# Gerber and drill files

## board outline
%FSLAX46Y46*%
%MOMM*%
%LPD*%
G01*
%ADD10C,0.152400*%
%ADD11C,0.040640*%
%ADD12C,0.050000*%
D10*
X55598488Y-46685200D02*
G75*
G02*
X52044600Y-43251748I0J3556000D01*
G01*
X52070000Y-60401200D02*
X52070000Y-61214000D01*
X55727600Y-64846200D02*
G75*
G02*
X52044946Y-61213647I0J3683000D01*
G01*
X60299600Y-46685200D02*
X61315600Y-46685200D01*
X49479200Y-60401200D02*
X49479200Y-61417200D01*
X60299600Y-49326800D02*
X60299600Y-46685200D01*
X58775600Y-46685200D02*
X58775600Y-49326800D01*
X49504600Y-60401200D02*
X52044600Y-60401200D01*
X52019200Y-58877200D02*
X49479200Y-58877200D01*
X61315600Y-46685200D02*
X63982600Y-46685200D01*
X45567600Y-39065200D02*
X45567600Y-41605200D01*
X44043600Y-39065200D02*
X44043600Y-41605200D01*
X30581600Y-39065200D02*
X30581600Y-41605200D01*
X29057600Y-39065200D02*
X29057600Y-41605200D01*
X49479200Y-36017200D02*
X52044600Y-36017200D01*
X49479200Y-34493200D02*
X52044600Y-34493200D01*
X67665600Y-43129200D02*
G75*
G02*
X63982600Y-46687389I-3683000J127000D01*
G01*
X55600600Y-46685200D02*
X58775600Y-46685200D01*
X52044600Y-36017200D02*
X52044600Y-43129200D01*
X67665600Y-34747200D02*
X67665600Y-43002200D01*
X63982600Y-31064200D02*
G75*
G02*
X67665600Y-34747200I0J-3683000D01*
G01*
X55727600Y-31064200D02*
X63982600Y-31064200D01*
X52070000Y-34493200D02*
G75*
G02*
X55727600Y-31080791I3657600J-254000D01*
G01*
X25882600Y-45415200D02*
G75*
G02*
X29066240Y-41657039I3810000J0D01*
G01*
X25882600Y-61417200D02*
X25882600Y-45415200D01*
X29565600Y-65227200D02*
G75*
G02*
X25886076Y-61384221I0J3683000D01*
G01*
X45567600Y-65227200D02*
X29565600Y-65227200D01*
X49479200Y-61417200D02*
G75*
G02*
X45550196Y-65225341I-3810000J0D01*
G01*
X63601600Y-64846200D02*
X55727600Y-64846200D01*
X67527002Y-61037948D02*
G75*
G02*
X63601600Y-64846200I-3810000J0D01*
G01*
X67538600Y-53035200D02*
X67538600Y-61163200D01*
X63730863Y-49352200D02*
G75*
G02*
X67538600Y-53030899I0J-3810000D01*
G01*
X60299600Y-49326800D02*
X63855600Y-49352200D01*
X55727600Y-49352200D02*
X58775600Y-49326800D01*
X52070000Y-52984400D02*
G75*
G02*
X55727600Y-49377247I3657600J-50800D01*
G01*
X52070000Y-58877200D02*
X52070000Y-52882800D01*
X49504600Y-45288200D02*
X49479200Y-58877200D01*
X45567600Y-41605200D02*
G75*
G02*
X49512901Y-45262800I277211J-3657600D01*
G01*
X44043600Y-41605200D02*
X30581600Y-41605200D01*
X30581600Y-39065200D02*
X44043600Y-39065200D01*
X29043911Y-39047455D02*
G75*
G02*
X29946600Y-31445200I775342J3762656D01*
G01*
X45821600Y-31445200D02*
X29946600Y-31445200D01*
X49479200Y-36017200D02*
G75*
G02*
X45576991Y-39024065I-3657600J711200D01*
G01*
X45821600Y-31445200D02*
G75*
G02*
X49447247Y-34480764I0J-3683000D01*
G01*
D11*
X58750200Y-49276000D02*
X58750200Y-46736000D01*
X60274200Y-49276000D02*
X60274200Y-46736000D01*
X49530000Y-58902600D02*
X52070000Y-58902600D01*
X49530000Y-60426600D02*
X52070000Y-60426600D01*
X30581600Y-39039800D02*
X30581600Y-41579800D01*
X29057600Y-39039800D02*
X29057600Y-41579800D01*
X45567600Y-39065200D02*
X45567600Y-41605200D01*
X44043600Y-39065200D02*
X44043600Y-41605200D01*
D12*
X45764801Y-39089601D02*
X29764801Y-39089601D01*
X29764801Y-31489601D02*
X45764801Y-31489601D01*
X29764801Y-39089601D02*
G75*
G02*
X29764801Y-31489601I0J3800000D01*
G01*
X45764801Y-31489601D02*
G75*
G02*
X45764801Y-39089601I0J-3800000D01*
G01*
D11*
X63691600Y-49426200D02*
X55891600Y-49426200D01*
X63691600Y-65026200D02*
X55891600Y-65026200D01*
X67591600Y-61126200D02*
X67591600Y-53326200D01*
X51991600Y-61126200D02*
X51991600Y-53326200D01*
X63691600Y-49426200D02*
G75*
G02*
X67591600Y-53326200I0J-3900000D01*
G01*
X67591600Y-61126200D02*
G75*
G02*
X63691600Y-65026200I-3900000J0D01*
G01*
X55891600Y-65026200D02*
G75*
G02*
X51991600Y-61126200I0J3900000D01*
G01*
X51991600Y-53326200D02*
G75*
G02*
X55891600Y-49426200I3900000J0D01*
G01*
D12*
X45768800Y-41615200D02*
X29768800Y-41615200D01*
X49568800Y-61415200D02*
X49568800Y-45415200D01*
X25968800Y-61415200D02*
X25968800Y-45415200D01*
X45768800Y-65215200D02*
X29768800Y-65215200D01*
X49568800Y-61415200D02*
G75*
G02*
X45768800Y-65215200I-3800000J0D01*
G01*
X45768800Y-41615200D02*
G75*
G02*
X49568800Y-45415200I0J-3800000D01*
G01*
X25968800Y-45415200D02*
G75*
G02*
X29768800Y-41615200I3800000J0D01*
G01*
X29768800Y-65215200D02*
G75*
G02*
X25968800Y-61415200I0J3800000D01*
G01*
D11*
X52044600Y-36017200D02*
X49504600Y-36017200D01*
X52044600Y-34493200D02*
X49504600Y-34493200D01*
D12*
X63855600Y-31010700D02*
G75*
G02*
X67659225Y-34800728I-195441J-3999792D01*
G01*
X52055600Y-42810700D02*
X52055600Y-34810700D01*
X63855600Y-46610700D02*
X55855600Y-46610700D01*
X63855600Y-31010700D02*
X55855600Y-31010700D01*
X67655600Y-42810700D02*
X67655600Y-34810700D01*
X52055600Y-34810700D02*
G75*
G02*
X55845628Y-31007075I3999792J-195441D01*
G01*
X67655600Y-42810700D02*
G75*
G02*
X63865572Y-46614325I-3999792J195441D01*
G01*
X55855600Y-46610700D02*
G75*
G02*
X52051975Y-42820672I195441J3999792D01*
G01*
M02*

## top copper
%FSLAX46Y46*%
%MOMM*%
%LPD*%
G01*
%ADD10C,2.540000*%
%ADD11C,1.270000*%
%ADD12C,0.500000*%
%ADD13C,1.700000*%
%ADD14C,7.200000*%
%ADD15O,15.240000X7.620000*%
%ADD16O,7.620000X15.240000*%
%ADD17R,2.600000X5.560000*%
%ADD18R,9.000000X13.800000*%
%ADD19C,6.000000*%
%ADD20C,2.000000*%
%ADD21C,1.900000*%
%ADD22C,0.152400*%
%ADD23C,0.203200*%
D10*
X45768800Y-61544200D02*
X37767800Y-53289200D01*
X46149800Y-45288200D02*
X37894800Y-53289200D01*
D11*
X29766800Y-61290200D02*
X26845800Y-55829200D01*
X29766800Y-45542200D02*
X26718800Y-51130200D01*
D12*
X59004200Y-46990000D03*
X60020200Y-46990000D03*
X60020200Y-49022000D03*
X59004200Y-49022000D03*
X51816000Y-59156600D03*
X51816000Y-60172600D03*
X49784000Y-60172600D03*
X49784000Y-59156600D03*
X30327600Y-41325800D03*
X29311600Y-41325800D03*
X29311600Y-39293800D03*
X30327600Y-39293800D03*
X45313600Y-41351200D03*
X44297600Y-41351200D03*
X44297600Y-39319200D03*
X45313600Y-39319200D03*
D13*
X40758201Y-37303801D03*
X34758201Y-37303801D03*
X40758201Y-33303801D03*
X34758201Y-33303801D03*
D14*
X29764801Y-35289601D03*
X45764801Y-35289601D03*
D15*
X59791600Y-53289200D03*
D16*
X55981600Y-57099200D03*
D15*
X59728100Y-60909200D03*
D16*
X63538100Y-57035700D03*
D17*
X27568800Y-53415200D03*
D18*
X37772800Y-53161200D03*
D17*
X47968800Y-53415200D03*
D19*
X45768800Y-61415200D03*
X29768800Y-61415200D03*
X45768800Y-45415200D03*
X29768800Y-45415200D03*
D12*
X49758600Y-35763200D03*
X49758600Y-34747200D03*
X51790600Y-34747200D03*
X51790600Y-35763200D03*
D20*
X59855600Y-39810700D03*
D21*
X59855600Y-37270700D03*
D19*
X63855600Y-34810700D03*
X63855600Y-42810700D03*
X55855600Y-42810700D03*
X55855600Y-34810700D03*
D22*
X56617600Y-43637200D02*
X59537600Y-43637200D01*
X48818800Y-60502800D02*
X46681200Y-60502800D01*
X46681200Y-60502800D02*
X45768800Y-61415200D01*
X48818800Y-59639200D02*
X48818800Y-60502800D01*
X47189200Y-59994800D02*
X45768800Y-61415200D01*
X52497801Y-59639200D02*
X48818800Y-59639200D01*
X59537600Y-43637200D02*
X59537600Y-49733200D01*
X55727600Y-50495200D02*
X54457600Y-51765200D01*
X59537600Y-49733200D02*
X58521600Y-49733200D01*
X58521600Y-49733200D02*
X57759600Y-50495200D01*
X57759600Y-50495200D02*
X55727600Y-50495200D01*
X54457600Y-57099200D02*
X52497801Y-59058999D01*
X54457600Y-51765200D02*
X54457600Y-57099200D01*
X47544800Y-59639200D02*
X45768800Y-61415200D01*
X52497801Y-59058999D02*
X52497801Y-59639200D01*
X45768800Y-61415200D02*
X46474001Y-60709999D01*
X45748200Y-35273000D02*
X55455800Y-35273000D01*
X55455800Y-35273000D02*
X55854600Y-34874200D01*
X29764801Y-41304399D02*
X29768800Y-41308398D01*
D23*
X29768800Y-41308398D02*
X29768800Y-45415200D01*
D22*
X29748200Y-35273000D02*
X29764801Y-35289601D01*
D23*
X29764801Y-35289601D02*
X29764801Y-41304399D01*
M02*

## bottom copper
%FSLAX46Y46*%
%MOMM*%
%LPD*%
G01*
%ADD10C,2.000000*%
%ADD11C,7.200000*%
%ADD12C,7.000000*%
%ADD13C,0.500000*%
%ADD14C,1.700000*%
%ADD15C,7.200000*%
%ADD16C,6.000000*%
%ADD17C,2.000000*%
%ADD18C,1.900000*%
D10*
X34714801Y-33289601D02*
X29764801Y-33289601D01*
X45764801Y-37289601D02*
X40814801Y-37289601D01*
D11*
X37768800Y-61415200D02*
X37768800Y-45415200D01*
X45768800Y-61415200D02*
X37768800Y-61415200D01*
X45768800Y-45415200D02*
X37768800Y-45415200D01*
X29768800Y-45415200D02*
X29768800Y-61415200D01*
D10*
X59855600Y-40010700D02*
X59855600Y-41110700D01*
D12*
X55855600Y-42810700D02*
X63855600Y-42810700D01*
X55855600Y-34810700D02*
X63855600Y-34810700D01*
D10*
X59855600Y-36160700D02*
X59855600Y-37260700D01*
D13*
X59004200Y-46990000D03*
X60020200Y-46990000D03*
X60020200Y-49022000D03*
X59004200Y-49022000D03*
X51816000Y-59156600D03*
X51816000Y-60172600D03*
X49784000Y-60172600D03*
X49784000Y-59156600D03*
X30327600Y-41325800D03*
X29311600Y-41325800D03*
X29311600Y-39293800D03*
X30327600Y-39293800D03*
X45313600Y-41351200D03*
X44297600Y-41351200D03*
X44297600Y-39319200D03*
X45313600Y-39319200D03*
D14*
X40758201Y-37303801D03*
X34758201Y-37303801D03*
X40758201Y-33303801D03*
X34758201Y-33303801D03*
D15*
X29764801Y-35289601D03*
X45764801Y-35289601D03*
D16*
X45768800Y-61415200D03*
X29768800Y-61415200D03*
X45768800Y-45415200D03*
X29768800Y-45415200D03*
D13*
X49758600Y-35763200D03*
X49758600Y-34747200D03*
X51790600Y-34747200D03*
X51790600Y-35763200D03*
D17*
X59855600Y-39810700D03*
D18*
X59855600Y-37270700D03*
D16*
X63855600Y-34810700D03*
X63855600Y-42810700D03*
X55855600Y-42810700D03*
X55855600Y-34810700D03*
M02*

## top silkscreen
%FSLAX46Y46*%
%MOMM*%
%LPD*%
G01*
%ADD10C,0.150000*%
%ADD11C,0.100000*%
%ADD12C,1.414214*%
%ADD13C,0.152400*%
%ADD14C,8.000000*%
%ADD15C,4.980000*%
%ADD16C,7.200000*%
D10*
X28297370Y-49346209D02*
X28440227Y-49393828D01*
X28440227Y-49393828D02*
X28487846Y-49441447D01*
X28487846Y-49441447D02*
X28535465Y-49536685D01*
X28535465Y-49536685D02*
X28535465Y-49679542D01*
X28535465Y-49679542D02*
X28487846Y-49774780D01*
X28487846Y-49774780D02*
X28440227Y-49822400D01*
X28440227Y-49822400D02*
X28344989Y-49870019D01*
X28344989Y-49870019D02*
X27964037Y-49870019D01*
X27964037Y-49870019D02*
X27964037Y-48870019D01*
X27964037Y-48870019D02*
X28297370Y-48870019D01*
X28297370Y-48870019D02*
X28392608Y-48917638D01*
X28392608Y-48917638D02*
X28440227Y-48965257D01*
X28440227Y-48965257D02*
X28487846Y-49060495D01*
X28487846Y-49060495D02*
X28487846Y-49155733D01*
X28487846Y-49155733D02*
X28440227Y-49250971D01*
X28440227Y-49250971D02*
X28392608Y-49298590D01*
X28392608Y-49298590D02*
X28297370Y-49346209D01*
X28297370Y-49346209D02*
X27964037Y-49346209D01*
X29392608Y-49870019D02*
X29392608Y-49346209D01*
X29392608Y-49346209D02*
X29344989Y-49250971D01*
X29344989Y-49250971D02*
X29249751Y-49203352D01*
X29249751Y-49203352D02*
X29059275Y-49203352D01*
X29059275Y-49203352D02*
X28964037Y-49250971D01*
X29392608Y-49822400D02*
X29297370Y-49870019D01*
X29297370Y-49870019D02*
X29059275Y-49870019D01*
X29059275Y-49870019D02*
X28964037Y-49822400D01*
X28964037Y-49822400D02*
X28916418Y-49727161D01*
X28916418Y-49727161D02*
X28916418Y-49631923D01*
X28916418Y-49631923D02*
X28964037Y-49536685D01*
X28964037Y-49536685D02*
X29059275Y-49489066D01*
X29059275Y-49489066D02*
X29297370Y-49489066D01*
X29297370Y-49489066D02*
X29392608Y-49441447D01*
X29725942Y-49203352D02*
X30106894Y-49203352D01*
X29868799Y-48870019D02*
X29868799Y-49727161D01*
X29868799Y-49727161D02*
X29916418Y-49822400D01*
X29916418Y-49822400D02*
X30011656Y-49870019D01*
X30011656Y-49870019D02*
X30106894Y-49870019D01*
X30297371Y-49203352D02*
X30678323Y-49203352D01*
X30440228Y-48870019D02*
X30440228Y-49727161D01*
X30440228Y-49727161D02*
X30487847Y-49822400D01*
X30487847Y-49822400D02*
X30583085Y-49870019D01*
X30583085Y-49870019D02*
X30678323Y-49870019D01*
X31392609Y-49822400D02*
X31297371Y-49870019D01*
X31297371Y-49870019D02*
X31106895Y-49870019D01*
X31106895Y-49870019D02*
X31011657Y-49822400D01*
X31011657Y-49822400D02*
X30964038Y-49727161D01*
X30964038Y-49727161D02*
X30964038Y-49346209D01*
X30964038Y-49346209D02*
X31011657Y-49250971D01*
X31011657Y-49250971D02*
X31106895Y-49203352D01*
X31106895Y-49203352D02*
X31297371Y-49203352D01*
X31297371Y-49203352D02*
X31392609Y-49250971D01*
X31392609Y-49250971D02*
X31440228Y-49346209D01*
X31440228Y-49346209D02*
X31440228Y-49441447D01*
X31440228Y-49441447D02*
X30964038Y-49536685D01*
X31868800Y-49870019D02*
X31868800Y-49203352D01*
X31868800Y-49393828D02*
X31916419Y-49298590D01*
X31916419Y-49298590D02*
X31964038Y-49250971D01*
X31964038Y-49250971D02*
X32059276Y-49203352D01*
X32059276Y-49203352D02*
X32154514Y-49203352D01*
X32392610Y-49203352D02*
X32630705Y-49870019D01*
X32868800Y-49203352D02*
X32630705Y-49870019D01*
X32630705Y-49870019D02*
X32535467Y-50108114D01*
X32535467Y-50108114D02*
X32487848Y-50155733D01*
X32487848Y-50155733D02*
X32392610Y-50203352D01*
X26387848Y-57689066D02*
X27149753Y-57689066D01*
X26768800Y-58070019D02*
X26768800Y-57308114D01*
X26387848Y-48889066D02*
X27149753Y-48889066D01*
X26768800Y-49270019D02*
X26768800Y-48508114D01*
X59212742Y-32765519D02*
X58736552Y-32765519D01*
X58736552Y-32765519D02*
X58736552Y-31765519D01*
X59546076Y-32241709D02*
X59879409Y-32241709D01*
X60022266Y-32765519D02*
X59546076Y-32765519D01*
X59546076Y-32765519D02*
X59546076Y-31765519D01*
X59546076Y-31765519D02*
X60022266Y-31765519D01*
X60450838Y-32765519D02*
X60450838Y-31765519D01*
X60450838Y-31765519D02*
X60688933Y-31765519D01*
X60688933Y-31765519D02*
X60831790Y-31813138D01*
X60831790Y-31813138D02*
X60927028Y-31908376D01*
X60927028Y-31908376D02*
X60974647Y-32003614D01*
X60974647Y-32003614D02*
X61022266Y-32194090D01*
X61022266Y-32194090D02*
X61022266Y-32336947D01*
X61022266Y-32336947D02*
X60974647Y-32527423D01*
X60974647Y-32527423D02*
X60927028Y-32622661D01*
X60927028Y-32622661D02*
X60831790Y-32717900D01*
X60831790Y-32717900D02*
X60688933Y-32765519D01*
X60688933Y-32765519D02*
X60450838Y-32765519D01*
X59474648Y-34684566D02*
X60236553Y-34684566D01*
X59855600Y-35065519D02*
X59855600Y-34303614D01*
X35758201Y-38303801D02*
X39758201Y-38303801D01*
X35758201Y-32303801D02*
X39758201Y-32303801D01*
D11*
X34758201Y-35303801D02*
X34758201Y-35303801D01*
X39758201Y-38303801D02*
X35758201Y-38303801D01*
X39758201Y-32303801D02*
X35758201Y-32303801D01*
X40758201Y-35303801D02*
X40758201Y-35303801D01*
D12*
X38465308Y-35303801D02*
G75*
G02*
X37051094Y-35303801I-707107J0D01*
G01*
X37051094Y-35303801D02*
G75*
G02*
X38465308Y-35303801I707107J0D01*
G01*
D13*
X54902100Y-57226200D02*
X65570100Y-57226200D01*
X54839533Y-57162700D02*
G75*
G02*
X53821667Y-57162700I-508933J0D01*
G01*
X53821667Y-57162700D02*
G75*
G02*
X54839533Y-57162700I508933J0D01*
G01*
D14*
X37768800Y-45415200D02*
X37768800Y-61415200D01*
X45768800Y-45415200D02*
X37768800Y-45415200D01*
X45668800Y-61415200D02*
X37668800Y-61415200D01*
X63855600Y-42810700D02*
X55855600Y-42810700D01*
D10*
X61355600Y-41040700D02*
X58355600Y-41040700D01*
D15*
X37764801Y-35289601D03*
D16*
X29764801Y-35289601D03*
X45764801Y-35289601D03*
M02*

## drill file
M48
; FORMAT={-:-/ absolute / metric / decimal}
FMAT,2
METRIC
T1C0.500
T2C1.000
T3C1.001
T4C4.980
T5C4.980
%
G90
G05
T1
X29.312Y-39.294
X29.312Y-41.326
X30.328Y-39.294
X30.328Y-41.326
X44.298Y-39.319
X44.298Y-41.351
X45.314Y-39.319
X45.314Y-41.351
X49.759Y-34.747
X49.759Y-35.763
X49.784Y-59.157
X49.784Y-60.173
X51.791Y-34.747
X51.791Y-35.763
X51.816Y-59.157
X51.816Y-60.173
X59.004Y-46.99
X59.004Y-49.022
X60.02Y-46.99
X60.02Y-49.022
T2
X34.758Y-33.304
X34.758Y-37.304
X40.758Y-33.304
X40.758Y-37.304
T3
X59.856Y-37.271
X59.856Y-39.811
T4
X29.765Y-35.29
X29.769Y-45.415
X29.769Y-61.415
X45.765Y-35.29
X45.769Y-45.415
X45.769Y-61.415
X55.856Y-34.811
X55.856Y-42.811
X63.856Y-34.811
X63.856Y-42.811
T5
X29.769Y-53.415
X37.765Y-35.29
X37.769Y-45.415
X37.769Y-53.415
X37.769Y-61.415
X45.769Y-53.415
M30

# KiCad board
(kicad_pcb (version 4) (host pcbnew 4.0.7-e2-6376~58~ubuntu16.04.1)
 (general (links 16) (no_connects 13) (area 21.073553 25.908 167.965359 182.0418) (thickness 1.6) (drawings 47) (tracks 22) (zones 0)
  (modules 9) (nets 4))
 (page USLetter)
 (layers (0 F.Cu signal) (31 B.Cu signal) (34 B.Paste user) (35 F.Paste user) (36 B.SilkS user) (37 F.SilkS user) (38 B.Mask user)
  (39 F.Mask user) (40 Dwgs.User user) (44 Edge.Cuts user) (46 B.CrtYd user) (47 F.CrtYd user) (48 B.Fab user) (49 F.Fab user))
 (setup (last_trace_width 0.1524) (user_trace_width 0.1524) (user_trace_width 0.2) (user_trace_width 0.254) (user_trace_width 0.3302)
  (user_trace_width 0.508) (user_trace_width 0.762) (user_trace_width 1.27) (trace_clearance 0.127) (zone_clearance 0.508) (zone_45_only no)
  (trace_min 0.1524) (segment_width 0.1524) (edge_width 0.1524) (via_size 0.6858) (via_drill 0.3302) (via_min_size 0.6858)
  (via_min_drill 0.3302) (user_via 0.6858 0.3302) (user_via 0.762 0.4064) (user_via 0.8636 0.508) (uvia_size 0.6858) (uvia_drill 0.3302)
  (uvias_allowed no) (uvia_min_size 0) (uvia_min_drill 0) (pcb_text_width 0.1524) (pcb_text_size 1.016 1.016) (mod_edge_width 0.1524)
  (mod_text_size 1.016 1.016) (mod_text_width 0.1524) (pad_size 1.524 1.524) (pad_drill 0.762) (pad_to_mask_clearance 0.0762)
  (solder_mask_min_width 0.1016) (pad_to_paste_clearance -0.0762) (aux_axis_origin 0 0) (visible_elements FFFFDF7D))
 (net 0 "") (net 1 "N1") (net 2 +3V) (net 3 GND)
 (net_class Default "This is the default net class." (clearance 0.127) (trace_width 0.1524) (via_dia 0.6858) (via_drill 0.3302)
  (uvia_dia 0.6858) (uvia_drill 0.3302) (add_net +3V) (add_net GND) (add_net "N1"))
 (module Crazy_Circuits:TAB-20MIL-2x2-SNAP (layer F.Cu) (at 59.5122 48.006)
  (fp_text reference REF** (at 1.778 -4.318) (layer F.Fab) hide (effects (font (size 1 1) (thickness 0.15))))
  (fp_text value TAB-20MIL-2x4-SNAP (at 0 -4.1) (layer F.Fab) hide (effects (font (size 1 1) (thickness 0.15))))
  (fp_line (start -0.762 1.27) (end -0.762 -1.27) (layer Edge.Cuts) (width 0.04064))
  (fp_line (start 0.762 1.27) (end 0.762 -1.27) (layer Edge.Cuts) (width 0.04064))
  (pad 1 thru_hole circle (at -0.508 -1.016) (size 0.5 0.5) (drill 0.5) (layers *.Cu))
  (pad 1 thru_hole circle (at 0.508 -1.016) (size 0.5 0.5) (drill 0.5) (layers *.Cu))
  (pad 1 thru_hole circle (at 0.508 1.016) (size 0.5 0.5) (drill 0.5) (layers *.Cu))
  (pad 1 thru_hole circle (at -0.508 1.016) (size 0.5 0.5) (drill 0.5) (layers *.Cu)))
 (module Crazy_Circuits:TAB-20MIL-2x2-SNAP (layer F.Cu) (at 50.8 59.6646 270)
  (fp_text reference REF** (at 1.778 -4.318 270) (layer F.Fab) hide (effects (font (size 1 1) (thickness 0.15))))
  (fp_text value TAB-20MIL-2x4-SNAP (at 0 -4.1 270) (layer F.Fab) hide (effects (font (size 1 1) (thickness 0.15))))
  (fp_line (start -0.762 1.27) (end -0.762 -1.27) (layer Edge.Cuts) (width 0.04064))
  (fp_line (start 0.762 1.27) (end 0.762 -1.27) (layer Edge.Cuts) (width 0.04064))
  (pad 1 thru_hole circle (at -0.508 -1.016 270) (size 0.5 0.5) (drill 0.5) (layers *.Cu))
  (pad 1 thru_hole circle (at 0.508 -1.016 270) (size 0.5 0.5) (drill 0.5) (layers *.Cu))
  (pad 1 thru_hole circle (at 0.508 1.016 270) (size 0.5 0.5) (drill 0.5) (layers *.Cu))
  (pad 1 thru_hole circle (at -0.508 1.016 270) (size 0.5 0.5) (drill 0.5) (layers *.Cu)))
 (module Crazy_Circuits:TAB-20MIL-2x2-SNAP (layer F.Cu) (at 29.8196 40.3098 180)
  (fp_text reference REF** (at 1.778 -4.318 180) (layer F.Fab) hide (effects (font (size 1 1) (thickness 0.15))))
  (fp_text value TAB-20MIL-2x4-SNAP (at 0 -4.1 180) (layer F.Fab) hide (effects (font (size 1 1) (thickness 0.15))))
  (fp_line (start -0.762 1.27) (end -0.762 -1.27) (layer Edge.Cuts) (width 0.04064))
  (fp_line (start 0.762 1.27) (end 0.762 -1.27) (layer Edge.Cuts) (width 0.04064))
  (pad 1 thru_hole circle (at -0.508 -1.016 180) (size 0.5 0.5) (drill 0.5) (layers *.Cu))
  (pad 1 thru_hole circle (at 0.508 -1.016 180) (size 0.5 0.5) (drill 0.5) (layers *.Cu))
  (pad 1 thru_hole circle (at 0.508 1.016 180) (size 0.5 0.5) (drill 0.5) (layers *.Cu))
  (pad 1 thru_hole circle (at -0.508 1.016 180) (size 0.5 0.5) (drill 0.5) (layers *.Cu)))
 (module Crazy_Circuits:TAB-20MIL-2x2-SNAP (layer F.Cu) (at 44.8056 40.3352 180)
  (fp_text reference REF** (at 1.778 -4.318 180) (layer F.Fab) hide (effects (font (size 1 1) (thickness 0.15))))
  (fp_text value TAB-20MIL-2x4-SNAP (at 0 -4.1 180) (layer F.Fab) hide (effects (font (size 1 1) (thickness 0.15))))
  (fp_line (start -0.762 1.27) (end -0.762 -1.27) (layer Edge.Cuts) (width 0.04064))
  (fp_line (start 0.762 1.27) (end 0.762 -1.27) (layer Edge.Cuts) (width 0.04064))
  (pad 1 thru_hole circle (at -0.508 -1.016 180) (size 0.5 0.5) (drill 0.5) (layers *.Cu))
  (pad 1 thru_hole circle (at 0.508 -1.016 180) (size 0.5 0.5) (drill 0.5) (layers *.Cu))
  (pad 1 thru_hole circle (at 0.508 1.016 180) (size 0.5 0.5) (drill 0.5) (layers *.Cu))
  (pad 1 thru_hole circle (at -0.508 1.016 180) (size 0.5 0.5) (drill 0.5) (layers *.Cu)))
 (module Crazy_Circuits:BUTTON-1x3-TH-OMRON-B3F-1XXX (layer F.Cu) (at 29.764801 35.289601)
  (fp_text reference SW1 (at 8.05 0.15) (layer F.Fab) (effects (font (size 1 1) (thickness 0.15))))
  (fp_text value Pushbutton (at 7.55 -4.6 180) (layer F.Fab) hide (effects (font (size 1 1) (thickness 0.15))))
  (fp_line (start 16 3.8) (end 0 3.8) (layer Edge.Cuts) (width 0.05))
  (fp_line (start 0 -3.8) (end 16 -3.8) (layer Edge.Cuts) (width 0.05))
  (fp_arc (start 0 0) (end 0 3.8) (angle 180) (layer Edge.Cuts) (width 0.05)) (fp_line (start 4.95 -2) (end 0 -2) (layer B.Cu) (width 2))
  (fp_line (start 5.9934 3.0142) (end 9.9934 3.0142) (layer F.SilkS) (width 0.15))
  (fp_line (start 5.9934 -2.9858) (end 9.9934 -2.9858) (layer F.SilkS) (width 0.15))
  (fp_line (start 4.9934 0.0142) (end 4.9934 0.0142) (layer F.SilkS) (width 0))
  (fp_line (start 9.9934 3.0142) (end 5.9934 3.0142) (layer F.SilkS) (width 0))
  (fp_line (start 9.9934 -2.9858) (end 5.9934 -2.9858) (layer F.SilkS) (width 0))
  (fp_line (start 10.9934 0.0142) (end 10.9934 0.0142) (layer F.SilkS) (width 0))
  (fp_circle (center 7.9934 0.0142) (end 8.9934 1.0142) (layer F.SilkS) (width 0))
  (fp_line (start 16 2) (end 11.05 2) (layer B.Cu) (width 2))
  (fp_arc (start 16 0) (end 16 -3.8) (angle 180) (layer Edge.Cuts) (width 0.05))
  (pad 2 thru_hole circle (at 10.9934 2.0142) (size 1.7 1.7) (drill 1) (layers *.Cu *.Mask) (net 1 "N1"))
  (pad 2 thru_hole circle (at 4.9934 2.0142) (size 1.7 1.7) (drill 1) (layers *.Cu *.Mask) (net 1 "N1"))
  (pad 1 thru_hole circle (at 10.9934 -1.9858) (size 1.7 1.7) (drill 1) (layers *.Cu *.Mask) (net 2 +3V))
  (pad 1 thru_hole circle (at 4.9934 -1.9858) (size 1.7 1.7) (drill 1) (layers *.Cu *.Mask) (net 2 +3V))
  (pad "" np_thru_hole circle (at 8 0) (size 4.98 4.98) (drill 4.98) (layers *.Cu F.SilkS))
  (pad 1 thru_hole circle (at 0 0) (size 7.2 7.2) (drill 4.98) (layers *.Cu F.SilkS B.Mask) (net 2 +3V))
  (pad 2 thru_hole circle (at 16 0) (size 7.2 7.2) (drill 4.98) (layers *.Cu F.SilkS B.Mask) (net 1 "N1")))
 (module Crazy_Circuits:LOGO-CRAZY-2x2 (layer F.Cu) (at 59.7916 57.2262)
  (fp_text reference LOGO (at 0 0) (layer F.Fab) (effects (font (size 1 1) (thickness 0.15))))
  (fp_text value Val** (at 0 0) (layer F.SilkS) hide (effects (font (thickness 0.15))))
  (fp_line (start -4.8895 0) (end 5.7785 0) (layer F.SilkS) (width 0.1524))
  (fp_circle (center -5.461 -0.0635) (end -5.12358 0.3175) (layer F.SilkS) (width 0.1524))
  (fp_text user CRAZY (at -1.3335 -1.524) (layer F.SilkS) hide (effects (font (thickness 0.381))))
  (fp_line (start 3.9 -7.8) (end -3.9 -7.8) (layer Edge.Cuts) (width 0.04064))
  (fp_line (start 3.9 7.8) (end -3.9 7.8) (layer Edge.Cuts) (width 0.04064))
  (fp_line (start 7.8 3.9) (end 7.8 -3.9) (layer Edge.Cuts) (width 0.04064))
  (fp_line (start -7.8 3.9) (end -7.8 -3.9) (layer Edge.Cuts) (width 0.04064))
  (fp_arc (start 3.9 -3.9) (end 3.9 -7.8) (angle 90) (layer Edge.Cuts) (width 0.04064))
  (fp_arc (start 3.9 3.9) (end 7.8 3.9) (angle 90) (layer Edge.Cuts) (width 0.04064))
  (fp_arc (start -3.9 3.9) (end -3.9 7.8) (angle 90) (layer Edge.Cuts) (width 0.04064))
  (fp_arc (start -3.9 -3.9) (end -7.8 -3.9) (angle 90) (layer Edge.Cuts) (width 0.04064))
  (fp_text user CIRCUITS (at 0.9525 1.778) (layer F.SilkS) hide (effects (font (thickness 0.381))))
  (pad BG smd oval (at 0 -3.937) (size 15.24 7.62) (layers F.Cu))
  (pad BG smd oval (at -3.81 -0.127 90) (size 15.24 7.62) (layers F.Cu))
  (pad BG smd oval (at -0.0635 3.683 180) (size 15.24 7.62) (layers F.Cu))
  (pad BG smd oval (at 3.7465 -0.1905 270) (size 15.24 7.62) (layers F.Cu)))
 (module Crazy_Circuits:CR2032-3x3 (layer F.Cu) (at 45.7688 45.4152 180)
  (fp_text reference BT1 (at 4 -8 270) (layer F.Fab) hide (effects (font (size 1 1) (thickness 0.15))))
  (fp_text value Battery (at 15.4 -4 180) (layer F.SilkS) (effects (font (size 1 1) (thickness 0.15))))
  (fp_line (start 0 -16.129) (end 8.001 -7.874) (layer F.Cu) (width 2.54))
  (fp_line (start 0 3.8) (end 16 3.8) (layer Edge.Cuts) (width 0.05))
  (fp_line (start -3.8 -16) (end -3.8 0) (layer Edge.Cuts) (width 0.05))
  (fp_line (start 19.8 -16) (end 19.8 0) (layer Edge.Cuts) (width 0.05))
  (fp_line (start 0 -19.8) (end 16 -19.8) (layer Edge.Cuts) (width 0.05))
  (fp_arc (start 0 -16) (end -3.8 -16) (angle 90) (layer Edge.Cuts) (width 0.05))
  (fp_arc (start 0 0) (end 0 3.8) (angle 90) (layer Edge.Cuts) (width 0.05))
  (fp_arc (start 16 0) (end 19.8 0) (angle 90) (layer Edge.Cuts) (width 0.05))
  (fp_arc (start 16 -16) (end 16 -19.8) (angle 90) (layer Edge.Cuts) (width 0.05))
  (fp_line (start 8 0) (end 8 -16) (layer F.SilkS) (width 8)) (fp_line (start 8 -16) (end 8 0) (layer B.Cu) (width 7.2))
  (fp_line (start 0 -16) (end 8 -16) (layer B.Cu) (width 7.2)) (fp_line (start 0 0) (end 8 0) (layer B.Cu) (width 7.2))
  (fp_line (start 16 0) (end 16 -16) (layer B.Cu) (width 7.2))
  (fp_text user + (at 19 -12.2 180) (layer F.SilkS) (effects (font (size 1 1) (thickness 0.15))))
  (fp_line (start 0 0) (end 8 0) (layer F.SilkS) (width 8))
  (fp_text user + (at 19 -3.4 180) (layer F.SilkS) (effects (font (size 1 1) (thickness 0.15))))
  (fp_line (start 0.1 -16) (end 8.1 -16) (layer F.SilkS) (width 8))
  (fp_line (start -0.381 0.127) (end 7.874 -7.874) (layer F.Cu) (width 2.54))
  (fp_line (start 16.002 -15.875) (end 18.923 -10.414) (layer F.Cu) (width 1.27))
  (fp_line (start 16.002 -0.127) (end 19.05 -5.715) (layer F.Cu) (width 1.27))
  (pad "" np_thru_hole circle (at 8 -8 180) (size 4.98 4.98) (drill 4.98) (layers *.Cu B.Mask))
  (pad "" np_thru_hole circle (at 0 -8 180) (size 4.98 4.98) (drill 4.98) (layers *.Cu B.Mask))
  (pad "" np_thru_hole circle (at 16 -8 180) (size 4.98 4.98) (drill 4.98) (layers *.Cu B.Mask))
  (pad + smd rect (at 18.2 -8 180) (size 2.6 5.56) (layers F.Cu F.Paste F.Mask) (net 2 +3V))
  (pad GND smd rect (at 7.996 -7.746 180) (size 9 13.8) (layers F.Cu F.Paste F.Mask) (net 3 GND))
  (pad + smd rect (at -2.2 -8 180) (size 2.6 5.56) (layers F.Cu F.Paste F.Mask) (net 2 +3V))
  (pad GND thru_hole circle (at 0 -16 180) (size 6 6) (drill 4.98) (layers *.Cu B.Mask) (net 3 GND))
  (pad "" np_thru_hole circle (at 8 -16 180) (size 4.98 4.98) (drill 4.98) (layers *.Cu B.Mask))
  (pad + thru_hole circle (at 16 -16 180) (size 6 6) (drill 4.98) (layers *.Cu B.Mask) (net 2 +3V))
  (pad GND thru_hole circle (at 0 0 180) (size 6 6) (drill 4.98) (layers *.Cu B.Mask) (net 3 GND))
  (pad "" np_thru_hole circle (at 8 0 180) (size 4.98 4.98) (drill 4.98) (layers *.Cu B.Mask))
  (pad + thru_hole circle (at 16 0 180) (size 6 6) (drill 4.98) (layers *.Cu B.Mask) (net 2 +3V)))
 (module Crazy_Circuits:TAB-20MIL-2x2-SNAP (layer F.Cu) (at 50.7746 35.2552 90)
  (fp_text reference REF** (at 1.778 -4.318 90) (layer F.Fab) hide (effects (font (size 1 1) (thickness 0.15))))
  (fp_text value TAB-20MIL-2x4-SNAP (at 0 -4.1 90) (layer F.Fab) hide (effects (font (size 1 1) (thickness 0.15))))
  (fp_line (start -0.762 1.27) (end -0.762 -1.27) (layer Edge.Cuts) (width 0.04064))
  (fp_line (start 0.762 1.27) (end 0.762 -1.27) (layer Edge.Cuts) (width 0.04064))
  (pad 1 thru_hole circle (at -0.508 -1.016 90) (size 0.5 0.5) (drill 0.5) (layers *.Cu))
  (pad 1 thru_hole circle (at 0.508 -1.016 90) (size 0.5 0.5) (drill 0.5) (layers *.Cu))
  (pad 1 thru_hole circle (at 0.508 1.016 90) (size 0.5 0.5) (drill 0.5) (layers *.Cu))
  (pad 1 thru_hole circle (at -0.508 1.016 90) (size 0.5 0.5) (drill 0.5) (layers *.Cu)))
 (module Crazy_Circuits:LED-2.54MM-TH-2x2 (layer F.Cu) (at 63.8556 34.8107 180)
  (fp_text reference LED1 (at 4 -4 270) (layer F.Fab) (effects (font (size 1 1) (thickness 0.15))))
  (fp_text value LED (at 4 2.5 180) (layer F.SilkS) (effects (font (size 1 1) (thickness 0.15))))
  (fp_arc (start 0.195441 -0.199792) (end 0 3.8) (angle 84.2) (layer Edge.Cuts) (width 0.05))
  (fp_line (start 11.8 -8) (end 11.8 0) (layer Edge.Cuts) (width 0.05))
  (fp_line (start 0 -11.8) (end 8 -11.8) (layer Edge.Cuts) (width 0.05))
  (fp_line (start 0 3.8) (end 8 3.8) (layer Edge.Cuts) (width 0.05))
  (fp_line (start -3.8 -8) (end -3.8 0) (layer Edge.Cuts) (width 0.05)) (fp_line (start 4 -5.2) (end 4 -6.3) (layer B.Cu) (width 2))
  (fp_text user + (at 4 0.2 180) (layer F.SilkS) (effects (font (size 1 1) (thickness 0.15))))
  (fp_line (start 0 -8) (end 8 -8) (layer F.SilkS) (width 8))
  (fp_line (start 2.5 -6.23) (end 5.5 -6.23) (layer F.SilkS) (width 0.15)) (fp_line (start 8 -8) (end 0 -8) (layer B.Cu) (width 7))
  (fp_line (start 8 0) (end 0 0) (layer B.Cu) (width 7))
  (fp_line (start 4 -1.35) (end 4 -2.45) (layer B.Cu) (width 2))
  (fp_arc (start 7.800208 -0.195441) (end 11.8 0) (angle 84.2) (layer Edge.Cuts) (width 0.05))
  (fp_arc (start 0.199792 -7.804559) (end -3.8 -8) (angle 84.2) (layer Edge.Cuts) (width 0.05))
  (fp_arc (start 7.804559 -7.800208) (end 8 -11.8) (angle 84.2) (layer Edge.Cuts) (width 0.05))
  (pad - thru_hole circle (at 4 -5 180) (size 2 2) (drill 1.00076) (layers *.Cu *.Mask) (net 3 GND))
  (pad + thru_hole circle (at 4 -2.46 90) (size 1.9 1.9) (drill 1.00076) (layers *.Cu *.Mask) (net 1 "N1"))
  (pad + thru_hole circle (at 0 0 180) (size 6 6) (drill 4.98) (layers *.Cu F.Mask) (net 1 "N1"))
  (pad - thru_hole circle (at 0 -8 180) (size 6 6) (drill 4.98) (layers *.Cu F.Mask) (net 3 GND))
  (pad - thru_hole circle (at 8 -8 180) (size 6 6) (drill 4.98) (layers *.Cu F.Mask) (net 3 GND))
  (pad + thru_hole circle (at 8 0 180) (size 6 6) (drill 4.98) (layers *.Cu F.Mask) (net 1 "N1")))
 (gr_arc (start 55.598488 43.1292) (end 55.598488 46.6852) (angle 88.02506599) (layer Edge.Cuts) (width 0.1524))
 (gr_line (start 52.07 60.4012) (end 52.07 61.214) (layer Edge.Cuts) (width 0.1524))
 (gr_arc (start 55.7276 61.1632) (end 55.7276 64.8462) (angle 89.2151803) (layer Edge.Cuts) (width 0.1524))
 (gr_line (start 60.2996 46.6852) (end 61.3156 46.6852) (layer Edge.Cuts) (width 0.1524))
 (gr_line (start 49.4792 60.4012) (end 49.4792 61.4172) (layer Edge.Cuts) (width 0.1524))
 (gr_line (start 60.2996 49.3268) (end 60.2996 46.6852) (layer Edge.Cuts) (width 0.1524))
 (gr_line (start 58.7756 46.6852) (end 58.7756 49.3268) (layer Edge.Cuts) (width 0.1524))
 (gr_line (start 49.5046 60.4012) (end 52.0446 60.4012) (layer Edge.Cuts) (width 0.1524))
 (gr_line (start 52.0192 58.8772) (end 49.4792 58.8772) (layer Edge.Cuts) (width 0.1524))
 (gr_line (start 61.3156 46.6852) (end 63.9826 46.6852) (layer Edge.Cuts) (width 0.1524))
 (gr_line (start 45.5676 39.0652) (end 45.5676 41.6052) (layer Edge.Cuts) (width 0.1524))
 (gr_line (start 44.0436 39.0652) (end 44.0436 41.6052) (layer Edge.Cuts) (width 0.1524))
 (gr_line (start 30.5816 39.0652) (end 30.5816 41.6052) (layer Edge.Cuts) (width 0.1524))
 (gr_line (start 29.0576 39.0652) (end 29.0576 41.6052) (layer Edge.Cuts) (width 0.1524))
 (gr_line (start 49.4792 36.0172) (end 52.0446 36.0172) (layer Edge.Cuts) (width 0.1524))
 (gr_line (start 49.4792 34.4932) (end 52.0446 34.4932) (layer Edge.Cuts) (width 0.1524))
 (gr_arc (start 63.9826 43.0022) (end 67.6656 43.1292) (angle 88.02506599) (layer Edge.Cuts) (width 0.1524))
 (gr_line (start 55.6006 46.6852) (end 58.7756 46.6852) (layer Edge.Cuts) (width 0.1524))
 (gr_line (start 52.0446 36.0172) (end 52.0446 43.1292) (layer Edge.Cuts) (width 0.1524))
 (gr_line (start 67.6656 34.7472) (end 67.6656 43.0022) (layer Edge.Cuts) (width 0.1524))
 (gr_arc (start 63.9826 34.7472) (end 63.9826 31.0642) (angle 90) (layer Edge.Cuts) (width 0.1524))
 (gr_line (start 55.7276 31.0642) (end 63.9826 31.0642) (layer Edge.Cuts) (width 0.1524))
 (gr_arc (start 55.7276 34.7472) (end 52.07 34.4932) (angle 86.02750406) (layer Edge.Cuts) (width 0.1524))
 (gr_arc (start 29.6926 45.4152) (end 25.8826 45.4152) (angle 80.53767779) (layer Edge.Cuts) (width 0.1524))
 (gr_line (start 25.8826 61.4172) (end 25.8826 45.4152) (layer Edge.Cuts) (width 0.1524))
 (gr_arc (start 29.5656 61.5442) (end 29.5656 65.2272) (angle 92.48955292) (layer Edge.Cuts) (width 0.1524))
 (gr_line (start 45.5676 65.2272) (end 29.5656 65.2272) (layer Edge.Cuts) (width 0.1524))
 (gr_arc (start 45.6692 61.4172) (end 49.4792 61.4172) (angle 91.7899045) (layer Edge.Cuts) (width 0.1524))
 (gr_line (start 63.6016 64.8462) (end 55.7276 64.8462) (layer Edge.Cuts) (width 0.1524))
 (gr_arc (start 63.717002 61.037948) (end 67.527002 61.037948) (angle 91.73570459) (layer Edge.Cuts) (width 0.1524))
 (gr_line (start 67.5386 53.0352) (end 67.5386 61.1632) (layer Edge.Cuts) (width 0.1524))
 (gr_arc (start 63.730863 53.1622) (end 63.730863 49.3522) (angle 88.02506599) (layer Edge.Cuts) (width 0.1524))
 (gr_line (start 60.2996 49.3268) (end 63.8556 49.3522) (layer Edge.Cuts) (width 0.1524))
 (gr_line (start 55.7276 49.3522) (end 58.7756 49.3268) (layer Edge.Cuts) (width 0.1524))
 (gr_arc (start 55.7276 53.0352) (end 52.07 52.9844) (angle 89.20427645) (layer Edge.Cuts) (width 0.1524))
 (gr_line (start 52.07 58.8772) (end 52.07 52.8828) (layer Edge.Cuts) (width 0.1524))
 (gr_line (start 49.5046 45.2882) (end 49.4792 58.8772) (layer Edge.Cuts) (width 0.1524))
 (gr_arc (start 45.844811 45.2628) (end 45.5676 41.6052) (angle 94.33418445) (layer Edge.Cuts) (width 0.1524))
 (gr_line (start 44.0436 41.6052) (end 30.5816 41.6052) (layer Edge.Cuts) (width 0.1524))
 (gr_line (start 30.5816 39.0652) (end 44.0436 39.0652) (layer Edge.Cuts) (width 0.1524))
 (gr_arc (start 29.819253 35.284799) (end 29.043911 39.047455) (angle 170.256088) (layer Edge.Cuts) (width 0.1524))
 (gr_line (start 45.8216 31.4452) (end 29.9466 31.4452) (layer Edge.Cuts) (width 0.1524))
 (gr_arc (start 45.8216 35.306) (end 49.4792 36.0172) (angle 82.76048574) (layer Edge.Cuts) (width 0.1524))
 (gr_arc (start 45.8216 35.1282) (end 45.8216 31.4452) (angle 79.87534038) (layer Edge.Cuts) (width 0.1524))
 (segment (start 56.6176 43.6372) (end 59.5376 43.6372) (width 0.1524) (layer F.Cu) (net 3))
 (segment (start 48.8188 60.5028) (end 46.6812 60.5028) (width 0.1524) (layer F.Cu) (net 3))
 (segment (start 46.6812 60.5028) (end 45.7688 61.4152) (width 0.1524) (layer F.Cu) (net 3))
 (segment (start 48.8188 59.6392) (end 48.8188 60.5028) (width 0.1524) (layer F.Cu) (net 3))
 (segment (start 47.1892 59.9948) (end 45.7688 61.4152) (width 0.1524) (layer F.Cu) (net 3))
 (segment (start 52.497801 59.6392) (end 48.8188 59.6392) (width 0.1524) (layer F.Cu) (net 3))
 (segment (start 59.5376 43.6372) (end 59.5376 49.7332) (width 0.1524) (layer F.Cu) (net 3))
 (segment (start 55.7276 50.4952) (end 54.4576 51.7652) (width 0.1524) (layer F.Cu) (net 3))
 (segment (start 59.5376 49.7332) (end 58.5216 49.7332) (width 0.1524) (layer F.Cu) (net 3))
 (segment (start 58.5216 49.7332) (end 57.7596 50.4952) (width 0.1524) (layer F.Cu) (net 3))
 (segment (start 57.7596 50.4952) (end 55.7276 50.4952) (width 0.1524) (layer F.Cu) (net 3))
 (segment (start 54.4576 57.0992) (end 52.497801 59.058999) (width 0.1524) (layer F.Cu) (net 3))
 (segment (start 54.4576 51.7652) (end 54.4576 57.0992) (width 0.1524) (layer F.Cu) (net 3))
 (segment (start 47.5448 59.6392) (end 45.7688 61.4152) (width 0.1524) (layer F.Cu) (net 3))
 (segment (start 52.497801 59.058999) (end 52.497801 59.6392) (width 0.1524) (layer F.Cu) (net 3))
 (segment (start 45.7688 61.4152) (end 46.474001 60.709999) (width 0.1524) (layer F.Cu) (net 3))
 (segment (start 45.7482 35.273) (end 55.4558 35.273) (width 0.1524) (layer F.Cu) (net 1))
 (segment (start 55.4558 35.273) (end 55.8546 34.8742) (width 0.1524) (layer F.Cu) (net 1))
 (segment (start 29.764801 41.304399) (end 29.7688 41.308398) (width 0.1524) (layer F.Cu) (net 2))
 (segment (start 29.7688 41.308398) (end 29.7688 45.4152) (width 0.2032) (layer F.Cu) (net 2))
 (segment (start 29.7482 35.273) (end 29.764801 35.289601) (width 0.1524) (layer F.Cu) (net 2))
 (segment (start 29.764801 35.289601) (end 29.764801 41.304399) (width 0.2032) (layer F.Cu) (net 2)))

